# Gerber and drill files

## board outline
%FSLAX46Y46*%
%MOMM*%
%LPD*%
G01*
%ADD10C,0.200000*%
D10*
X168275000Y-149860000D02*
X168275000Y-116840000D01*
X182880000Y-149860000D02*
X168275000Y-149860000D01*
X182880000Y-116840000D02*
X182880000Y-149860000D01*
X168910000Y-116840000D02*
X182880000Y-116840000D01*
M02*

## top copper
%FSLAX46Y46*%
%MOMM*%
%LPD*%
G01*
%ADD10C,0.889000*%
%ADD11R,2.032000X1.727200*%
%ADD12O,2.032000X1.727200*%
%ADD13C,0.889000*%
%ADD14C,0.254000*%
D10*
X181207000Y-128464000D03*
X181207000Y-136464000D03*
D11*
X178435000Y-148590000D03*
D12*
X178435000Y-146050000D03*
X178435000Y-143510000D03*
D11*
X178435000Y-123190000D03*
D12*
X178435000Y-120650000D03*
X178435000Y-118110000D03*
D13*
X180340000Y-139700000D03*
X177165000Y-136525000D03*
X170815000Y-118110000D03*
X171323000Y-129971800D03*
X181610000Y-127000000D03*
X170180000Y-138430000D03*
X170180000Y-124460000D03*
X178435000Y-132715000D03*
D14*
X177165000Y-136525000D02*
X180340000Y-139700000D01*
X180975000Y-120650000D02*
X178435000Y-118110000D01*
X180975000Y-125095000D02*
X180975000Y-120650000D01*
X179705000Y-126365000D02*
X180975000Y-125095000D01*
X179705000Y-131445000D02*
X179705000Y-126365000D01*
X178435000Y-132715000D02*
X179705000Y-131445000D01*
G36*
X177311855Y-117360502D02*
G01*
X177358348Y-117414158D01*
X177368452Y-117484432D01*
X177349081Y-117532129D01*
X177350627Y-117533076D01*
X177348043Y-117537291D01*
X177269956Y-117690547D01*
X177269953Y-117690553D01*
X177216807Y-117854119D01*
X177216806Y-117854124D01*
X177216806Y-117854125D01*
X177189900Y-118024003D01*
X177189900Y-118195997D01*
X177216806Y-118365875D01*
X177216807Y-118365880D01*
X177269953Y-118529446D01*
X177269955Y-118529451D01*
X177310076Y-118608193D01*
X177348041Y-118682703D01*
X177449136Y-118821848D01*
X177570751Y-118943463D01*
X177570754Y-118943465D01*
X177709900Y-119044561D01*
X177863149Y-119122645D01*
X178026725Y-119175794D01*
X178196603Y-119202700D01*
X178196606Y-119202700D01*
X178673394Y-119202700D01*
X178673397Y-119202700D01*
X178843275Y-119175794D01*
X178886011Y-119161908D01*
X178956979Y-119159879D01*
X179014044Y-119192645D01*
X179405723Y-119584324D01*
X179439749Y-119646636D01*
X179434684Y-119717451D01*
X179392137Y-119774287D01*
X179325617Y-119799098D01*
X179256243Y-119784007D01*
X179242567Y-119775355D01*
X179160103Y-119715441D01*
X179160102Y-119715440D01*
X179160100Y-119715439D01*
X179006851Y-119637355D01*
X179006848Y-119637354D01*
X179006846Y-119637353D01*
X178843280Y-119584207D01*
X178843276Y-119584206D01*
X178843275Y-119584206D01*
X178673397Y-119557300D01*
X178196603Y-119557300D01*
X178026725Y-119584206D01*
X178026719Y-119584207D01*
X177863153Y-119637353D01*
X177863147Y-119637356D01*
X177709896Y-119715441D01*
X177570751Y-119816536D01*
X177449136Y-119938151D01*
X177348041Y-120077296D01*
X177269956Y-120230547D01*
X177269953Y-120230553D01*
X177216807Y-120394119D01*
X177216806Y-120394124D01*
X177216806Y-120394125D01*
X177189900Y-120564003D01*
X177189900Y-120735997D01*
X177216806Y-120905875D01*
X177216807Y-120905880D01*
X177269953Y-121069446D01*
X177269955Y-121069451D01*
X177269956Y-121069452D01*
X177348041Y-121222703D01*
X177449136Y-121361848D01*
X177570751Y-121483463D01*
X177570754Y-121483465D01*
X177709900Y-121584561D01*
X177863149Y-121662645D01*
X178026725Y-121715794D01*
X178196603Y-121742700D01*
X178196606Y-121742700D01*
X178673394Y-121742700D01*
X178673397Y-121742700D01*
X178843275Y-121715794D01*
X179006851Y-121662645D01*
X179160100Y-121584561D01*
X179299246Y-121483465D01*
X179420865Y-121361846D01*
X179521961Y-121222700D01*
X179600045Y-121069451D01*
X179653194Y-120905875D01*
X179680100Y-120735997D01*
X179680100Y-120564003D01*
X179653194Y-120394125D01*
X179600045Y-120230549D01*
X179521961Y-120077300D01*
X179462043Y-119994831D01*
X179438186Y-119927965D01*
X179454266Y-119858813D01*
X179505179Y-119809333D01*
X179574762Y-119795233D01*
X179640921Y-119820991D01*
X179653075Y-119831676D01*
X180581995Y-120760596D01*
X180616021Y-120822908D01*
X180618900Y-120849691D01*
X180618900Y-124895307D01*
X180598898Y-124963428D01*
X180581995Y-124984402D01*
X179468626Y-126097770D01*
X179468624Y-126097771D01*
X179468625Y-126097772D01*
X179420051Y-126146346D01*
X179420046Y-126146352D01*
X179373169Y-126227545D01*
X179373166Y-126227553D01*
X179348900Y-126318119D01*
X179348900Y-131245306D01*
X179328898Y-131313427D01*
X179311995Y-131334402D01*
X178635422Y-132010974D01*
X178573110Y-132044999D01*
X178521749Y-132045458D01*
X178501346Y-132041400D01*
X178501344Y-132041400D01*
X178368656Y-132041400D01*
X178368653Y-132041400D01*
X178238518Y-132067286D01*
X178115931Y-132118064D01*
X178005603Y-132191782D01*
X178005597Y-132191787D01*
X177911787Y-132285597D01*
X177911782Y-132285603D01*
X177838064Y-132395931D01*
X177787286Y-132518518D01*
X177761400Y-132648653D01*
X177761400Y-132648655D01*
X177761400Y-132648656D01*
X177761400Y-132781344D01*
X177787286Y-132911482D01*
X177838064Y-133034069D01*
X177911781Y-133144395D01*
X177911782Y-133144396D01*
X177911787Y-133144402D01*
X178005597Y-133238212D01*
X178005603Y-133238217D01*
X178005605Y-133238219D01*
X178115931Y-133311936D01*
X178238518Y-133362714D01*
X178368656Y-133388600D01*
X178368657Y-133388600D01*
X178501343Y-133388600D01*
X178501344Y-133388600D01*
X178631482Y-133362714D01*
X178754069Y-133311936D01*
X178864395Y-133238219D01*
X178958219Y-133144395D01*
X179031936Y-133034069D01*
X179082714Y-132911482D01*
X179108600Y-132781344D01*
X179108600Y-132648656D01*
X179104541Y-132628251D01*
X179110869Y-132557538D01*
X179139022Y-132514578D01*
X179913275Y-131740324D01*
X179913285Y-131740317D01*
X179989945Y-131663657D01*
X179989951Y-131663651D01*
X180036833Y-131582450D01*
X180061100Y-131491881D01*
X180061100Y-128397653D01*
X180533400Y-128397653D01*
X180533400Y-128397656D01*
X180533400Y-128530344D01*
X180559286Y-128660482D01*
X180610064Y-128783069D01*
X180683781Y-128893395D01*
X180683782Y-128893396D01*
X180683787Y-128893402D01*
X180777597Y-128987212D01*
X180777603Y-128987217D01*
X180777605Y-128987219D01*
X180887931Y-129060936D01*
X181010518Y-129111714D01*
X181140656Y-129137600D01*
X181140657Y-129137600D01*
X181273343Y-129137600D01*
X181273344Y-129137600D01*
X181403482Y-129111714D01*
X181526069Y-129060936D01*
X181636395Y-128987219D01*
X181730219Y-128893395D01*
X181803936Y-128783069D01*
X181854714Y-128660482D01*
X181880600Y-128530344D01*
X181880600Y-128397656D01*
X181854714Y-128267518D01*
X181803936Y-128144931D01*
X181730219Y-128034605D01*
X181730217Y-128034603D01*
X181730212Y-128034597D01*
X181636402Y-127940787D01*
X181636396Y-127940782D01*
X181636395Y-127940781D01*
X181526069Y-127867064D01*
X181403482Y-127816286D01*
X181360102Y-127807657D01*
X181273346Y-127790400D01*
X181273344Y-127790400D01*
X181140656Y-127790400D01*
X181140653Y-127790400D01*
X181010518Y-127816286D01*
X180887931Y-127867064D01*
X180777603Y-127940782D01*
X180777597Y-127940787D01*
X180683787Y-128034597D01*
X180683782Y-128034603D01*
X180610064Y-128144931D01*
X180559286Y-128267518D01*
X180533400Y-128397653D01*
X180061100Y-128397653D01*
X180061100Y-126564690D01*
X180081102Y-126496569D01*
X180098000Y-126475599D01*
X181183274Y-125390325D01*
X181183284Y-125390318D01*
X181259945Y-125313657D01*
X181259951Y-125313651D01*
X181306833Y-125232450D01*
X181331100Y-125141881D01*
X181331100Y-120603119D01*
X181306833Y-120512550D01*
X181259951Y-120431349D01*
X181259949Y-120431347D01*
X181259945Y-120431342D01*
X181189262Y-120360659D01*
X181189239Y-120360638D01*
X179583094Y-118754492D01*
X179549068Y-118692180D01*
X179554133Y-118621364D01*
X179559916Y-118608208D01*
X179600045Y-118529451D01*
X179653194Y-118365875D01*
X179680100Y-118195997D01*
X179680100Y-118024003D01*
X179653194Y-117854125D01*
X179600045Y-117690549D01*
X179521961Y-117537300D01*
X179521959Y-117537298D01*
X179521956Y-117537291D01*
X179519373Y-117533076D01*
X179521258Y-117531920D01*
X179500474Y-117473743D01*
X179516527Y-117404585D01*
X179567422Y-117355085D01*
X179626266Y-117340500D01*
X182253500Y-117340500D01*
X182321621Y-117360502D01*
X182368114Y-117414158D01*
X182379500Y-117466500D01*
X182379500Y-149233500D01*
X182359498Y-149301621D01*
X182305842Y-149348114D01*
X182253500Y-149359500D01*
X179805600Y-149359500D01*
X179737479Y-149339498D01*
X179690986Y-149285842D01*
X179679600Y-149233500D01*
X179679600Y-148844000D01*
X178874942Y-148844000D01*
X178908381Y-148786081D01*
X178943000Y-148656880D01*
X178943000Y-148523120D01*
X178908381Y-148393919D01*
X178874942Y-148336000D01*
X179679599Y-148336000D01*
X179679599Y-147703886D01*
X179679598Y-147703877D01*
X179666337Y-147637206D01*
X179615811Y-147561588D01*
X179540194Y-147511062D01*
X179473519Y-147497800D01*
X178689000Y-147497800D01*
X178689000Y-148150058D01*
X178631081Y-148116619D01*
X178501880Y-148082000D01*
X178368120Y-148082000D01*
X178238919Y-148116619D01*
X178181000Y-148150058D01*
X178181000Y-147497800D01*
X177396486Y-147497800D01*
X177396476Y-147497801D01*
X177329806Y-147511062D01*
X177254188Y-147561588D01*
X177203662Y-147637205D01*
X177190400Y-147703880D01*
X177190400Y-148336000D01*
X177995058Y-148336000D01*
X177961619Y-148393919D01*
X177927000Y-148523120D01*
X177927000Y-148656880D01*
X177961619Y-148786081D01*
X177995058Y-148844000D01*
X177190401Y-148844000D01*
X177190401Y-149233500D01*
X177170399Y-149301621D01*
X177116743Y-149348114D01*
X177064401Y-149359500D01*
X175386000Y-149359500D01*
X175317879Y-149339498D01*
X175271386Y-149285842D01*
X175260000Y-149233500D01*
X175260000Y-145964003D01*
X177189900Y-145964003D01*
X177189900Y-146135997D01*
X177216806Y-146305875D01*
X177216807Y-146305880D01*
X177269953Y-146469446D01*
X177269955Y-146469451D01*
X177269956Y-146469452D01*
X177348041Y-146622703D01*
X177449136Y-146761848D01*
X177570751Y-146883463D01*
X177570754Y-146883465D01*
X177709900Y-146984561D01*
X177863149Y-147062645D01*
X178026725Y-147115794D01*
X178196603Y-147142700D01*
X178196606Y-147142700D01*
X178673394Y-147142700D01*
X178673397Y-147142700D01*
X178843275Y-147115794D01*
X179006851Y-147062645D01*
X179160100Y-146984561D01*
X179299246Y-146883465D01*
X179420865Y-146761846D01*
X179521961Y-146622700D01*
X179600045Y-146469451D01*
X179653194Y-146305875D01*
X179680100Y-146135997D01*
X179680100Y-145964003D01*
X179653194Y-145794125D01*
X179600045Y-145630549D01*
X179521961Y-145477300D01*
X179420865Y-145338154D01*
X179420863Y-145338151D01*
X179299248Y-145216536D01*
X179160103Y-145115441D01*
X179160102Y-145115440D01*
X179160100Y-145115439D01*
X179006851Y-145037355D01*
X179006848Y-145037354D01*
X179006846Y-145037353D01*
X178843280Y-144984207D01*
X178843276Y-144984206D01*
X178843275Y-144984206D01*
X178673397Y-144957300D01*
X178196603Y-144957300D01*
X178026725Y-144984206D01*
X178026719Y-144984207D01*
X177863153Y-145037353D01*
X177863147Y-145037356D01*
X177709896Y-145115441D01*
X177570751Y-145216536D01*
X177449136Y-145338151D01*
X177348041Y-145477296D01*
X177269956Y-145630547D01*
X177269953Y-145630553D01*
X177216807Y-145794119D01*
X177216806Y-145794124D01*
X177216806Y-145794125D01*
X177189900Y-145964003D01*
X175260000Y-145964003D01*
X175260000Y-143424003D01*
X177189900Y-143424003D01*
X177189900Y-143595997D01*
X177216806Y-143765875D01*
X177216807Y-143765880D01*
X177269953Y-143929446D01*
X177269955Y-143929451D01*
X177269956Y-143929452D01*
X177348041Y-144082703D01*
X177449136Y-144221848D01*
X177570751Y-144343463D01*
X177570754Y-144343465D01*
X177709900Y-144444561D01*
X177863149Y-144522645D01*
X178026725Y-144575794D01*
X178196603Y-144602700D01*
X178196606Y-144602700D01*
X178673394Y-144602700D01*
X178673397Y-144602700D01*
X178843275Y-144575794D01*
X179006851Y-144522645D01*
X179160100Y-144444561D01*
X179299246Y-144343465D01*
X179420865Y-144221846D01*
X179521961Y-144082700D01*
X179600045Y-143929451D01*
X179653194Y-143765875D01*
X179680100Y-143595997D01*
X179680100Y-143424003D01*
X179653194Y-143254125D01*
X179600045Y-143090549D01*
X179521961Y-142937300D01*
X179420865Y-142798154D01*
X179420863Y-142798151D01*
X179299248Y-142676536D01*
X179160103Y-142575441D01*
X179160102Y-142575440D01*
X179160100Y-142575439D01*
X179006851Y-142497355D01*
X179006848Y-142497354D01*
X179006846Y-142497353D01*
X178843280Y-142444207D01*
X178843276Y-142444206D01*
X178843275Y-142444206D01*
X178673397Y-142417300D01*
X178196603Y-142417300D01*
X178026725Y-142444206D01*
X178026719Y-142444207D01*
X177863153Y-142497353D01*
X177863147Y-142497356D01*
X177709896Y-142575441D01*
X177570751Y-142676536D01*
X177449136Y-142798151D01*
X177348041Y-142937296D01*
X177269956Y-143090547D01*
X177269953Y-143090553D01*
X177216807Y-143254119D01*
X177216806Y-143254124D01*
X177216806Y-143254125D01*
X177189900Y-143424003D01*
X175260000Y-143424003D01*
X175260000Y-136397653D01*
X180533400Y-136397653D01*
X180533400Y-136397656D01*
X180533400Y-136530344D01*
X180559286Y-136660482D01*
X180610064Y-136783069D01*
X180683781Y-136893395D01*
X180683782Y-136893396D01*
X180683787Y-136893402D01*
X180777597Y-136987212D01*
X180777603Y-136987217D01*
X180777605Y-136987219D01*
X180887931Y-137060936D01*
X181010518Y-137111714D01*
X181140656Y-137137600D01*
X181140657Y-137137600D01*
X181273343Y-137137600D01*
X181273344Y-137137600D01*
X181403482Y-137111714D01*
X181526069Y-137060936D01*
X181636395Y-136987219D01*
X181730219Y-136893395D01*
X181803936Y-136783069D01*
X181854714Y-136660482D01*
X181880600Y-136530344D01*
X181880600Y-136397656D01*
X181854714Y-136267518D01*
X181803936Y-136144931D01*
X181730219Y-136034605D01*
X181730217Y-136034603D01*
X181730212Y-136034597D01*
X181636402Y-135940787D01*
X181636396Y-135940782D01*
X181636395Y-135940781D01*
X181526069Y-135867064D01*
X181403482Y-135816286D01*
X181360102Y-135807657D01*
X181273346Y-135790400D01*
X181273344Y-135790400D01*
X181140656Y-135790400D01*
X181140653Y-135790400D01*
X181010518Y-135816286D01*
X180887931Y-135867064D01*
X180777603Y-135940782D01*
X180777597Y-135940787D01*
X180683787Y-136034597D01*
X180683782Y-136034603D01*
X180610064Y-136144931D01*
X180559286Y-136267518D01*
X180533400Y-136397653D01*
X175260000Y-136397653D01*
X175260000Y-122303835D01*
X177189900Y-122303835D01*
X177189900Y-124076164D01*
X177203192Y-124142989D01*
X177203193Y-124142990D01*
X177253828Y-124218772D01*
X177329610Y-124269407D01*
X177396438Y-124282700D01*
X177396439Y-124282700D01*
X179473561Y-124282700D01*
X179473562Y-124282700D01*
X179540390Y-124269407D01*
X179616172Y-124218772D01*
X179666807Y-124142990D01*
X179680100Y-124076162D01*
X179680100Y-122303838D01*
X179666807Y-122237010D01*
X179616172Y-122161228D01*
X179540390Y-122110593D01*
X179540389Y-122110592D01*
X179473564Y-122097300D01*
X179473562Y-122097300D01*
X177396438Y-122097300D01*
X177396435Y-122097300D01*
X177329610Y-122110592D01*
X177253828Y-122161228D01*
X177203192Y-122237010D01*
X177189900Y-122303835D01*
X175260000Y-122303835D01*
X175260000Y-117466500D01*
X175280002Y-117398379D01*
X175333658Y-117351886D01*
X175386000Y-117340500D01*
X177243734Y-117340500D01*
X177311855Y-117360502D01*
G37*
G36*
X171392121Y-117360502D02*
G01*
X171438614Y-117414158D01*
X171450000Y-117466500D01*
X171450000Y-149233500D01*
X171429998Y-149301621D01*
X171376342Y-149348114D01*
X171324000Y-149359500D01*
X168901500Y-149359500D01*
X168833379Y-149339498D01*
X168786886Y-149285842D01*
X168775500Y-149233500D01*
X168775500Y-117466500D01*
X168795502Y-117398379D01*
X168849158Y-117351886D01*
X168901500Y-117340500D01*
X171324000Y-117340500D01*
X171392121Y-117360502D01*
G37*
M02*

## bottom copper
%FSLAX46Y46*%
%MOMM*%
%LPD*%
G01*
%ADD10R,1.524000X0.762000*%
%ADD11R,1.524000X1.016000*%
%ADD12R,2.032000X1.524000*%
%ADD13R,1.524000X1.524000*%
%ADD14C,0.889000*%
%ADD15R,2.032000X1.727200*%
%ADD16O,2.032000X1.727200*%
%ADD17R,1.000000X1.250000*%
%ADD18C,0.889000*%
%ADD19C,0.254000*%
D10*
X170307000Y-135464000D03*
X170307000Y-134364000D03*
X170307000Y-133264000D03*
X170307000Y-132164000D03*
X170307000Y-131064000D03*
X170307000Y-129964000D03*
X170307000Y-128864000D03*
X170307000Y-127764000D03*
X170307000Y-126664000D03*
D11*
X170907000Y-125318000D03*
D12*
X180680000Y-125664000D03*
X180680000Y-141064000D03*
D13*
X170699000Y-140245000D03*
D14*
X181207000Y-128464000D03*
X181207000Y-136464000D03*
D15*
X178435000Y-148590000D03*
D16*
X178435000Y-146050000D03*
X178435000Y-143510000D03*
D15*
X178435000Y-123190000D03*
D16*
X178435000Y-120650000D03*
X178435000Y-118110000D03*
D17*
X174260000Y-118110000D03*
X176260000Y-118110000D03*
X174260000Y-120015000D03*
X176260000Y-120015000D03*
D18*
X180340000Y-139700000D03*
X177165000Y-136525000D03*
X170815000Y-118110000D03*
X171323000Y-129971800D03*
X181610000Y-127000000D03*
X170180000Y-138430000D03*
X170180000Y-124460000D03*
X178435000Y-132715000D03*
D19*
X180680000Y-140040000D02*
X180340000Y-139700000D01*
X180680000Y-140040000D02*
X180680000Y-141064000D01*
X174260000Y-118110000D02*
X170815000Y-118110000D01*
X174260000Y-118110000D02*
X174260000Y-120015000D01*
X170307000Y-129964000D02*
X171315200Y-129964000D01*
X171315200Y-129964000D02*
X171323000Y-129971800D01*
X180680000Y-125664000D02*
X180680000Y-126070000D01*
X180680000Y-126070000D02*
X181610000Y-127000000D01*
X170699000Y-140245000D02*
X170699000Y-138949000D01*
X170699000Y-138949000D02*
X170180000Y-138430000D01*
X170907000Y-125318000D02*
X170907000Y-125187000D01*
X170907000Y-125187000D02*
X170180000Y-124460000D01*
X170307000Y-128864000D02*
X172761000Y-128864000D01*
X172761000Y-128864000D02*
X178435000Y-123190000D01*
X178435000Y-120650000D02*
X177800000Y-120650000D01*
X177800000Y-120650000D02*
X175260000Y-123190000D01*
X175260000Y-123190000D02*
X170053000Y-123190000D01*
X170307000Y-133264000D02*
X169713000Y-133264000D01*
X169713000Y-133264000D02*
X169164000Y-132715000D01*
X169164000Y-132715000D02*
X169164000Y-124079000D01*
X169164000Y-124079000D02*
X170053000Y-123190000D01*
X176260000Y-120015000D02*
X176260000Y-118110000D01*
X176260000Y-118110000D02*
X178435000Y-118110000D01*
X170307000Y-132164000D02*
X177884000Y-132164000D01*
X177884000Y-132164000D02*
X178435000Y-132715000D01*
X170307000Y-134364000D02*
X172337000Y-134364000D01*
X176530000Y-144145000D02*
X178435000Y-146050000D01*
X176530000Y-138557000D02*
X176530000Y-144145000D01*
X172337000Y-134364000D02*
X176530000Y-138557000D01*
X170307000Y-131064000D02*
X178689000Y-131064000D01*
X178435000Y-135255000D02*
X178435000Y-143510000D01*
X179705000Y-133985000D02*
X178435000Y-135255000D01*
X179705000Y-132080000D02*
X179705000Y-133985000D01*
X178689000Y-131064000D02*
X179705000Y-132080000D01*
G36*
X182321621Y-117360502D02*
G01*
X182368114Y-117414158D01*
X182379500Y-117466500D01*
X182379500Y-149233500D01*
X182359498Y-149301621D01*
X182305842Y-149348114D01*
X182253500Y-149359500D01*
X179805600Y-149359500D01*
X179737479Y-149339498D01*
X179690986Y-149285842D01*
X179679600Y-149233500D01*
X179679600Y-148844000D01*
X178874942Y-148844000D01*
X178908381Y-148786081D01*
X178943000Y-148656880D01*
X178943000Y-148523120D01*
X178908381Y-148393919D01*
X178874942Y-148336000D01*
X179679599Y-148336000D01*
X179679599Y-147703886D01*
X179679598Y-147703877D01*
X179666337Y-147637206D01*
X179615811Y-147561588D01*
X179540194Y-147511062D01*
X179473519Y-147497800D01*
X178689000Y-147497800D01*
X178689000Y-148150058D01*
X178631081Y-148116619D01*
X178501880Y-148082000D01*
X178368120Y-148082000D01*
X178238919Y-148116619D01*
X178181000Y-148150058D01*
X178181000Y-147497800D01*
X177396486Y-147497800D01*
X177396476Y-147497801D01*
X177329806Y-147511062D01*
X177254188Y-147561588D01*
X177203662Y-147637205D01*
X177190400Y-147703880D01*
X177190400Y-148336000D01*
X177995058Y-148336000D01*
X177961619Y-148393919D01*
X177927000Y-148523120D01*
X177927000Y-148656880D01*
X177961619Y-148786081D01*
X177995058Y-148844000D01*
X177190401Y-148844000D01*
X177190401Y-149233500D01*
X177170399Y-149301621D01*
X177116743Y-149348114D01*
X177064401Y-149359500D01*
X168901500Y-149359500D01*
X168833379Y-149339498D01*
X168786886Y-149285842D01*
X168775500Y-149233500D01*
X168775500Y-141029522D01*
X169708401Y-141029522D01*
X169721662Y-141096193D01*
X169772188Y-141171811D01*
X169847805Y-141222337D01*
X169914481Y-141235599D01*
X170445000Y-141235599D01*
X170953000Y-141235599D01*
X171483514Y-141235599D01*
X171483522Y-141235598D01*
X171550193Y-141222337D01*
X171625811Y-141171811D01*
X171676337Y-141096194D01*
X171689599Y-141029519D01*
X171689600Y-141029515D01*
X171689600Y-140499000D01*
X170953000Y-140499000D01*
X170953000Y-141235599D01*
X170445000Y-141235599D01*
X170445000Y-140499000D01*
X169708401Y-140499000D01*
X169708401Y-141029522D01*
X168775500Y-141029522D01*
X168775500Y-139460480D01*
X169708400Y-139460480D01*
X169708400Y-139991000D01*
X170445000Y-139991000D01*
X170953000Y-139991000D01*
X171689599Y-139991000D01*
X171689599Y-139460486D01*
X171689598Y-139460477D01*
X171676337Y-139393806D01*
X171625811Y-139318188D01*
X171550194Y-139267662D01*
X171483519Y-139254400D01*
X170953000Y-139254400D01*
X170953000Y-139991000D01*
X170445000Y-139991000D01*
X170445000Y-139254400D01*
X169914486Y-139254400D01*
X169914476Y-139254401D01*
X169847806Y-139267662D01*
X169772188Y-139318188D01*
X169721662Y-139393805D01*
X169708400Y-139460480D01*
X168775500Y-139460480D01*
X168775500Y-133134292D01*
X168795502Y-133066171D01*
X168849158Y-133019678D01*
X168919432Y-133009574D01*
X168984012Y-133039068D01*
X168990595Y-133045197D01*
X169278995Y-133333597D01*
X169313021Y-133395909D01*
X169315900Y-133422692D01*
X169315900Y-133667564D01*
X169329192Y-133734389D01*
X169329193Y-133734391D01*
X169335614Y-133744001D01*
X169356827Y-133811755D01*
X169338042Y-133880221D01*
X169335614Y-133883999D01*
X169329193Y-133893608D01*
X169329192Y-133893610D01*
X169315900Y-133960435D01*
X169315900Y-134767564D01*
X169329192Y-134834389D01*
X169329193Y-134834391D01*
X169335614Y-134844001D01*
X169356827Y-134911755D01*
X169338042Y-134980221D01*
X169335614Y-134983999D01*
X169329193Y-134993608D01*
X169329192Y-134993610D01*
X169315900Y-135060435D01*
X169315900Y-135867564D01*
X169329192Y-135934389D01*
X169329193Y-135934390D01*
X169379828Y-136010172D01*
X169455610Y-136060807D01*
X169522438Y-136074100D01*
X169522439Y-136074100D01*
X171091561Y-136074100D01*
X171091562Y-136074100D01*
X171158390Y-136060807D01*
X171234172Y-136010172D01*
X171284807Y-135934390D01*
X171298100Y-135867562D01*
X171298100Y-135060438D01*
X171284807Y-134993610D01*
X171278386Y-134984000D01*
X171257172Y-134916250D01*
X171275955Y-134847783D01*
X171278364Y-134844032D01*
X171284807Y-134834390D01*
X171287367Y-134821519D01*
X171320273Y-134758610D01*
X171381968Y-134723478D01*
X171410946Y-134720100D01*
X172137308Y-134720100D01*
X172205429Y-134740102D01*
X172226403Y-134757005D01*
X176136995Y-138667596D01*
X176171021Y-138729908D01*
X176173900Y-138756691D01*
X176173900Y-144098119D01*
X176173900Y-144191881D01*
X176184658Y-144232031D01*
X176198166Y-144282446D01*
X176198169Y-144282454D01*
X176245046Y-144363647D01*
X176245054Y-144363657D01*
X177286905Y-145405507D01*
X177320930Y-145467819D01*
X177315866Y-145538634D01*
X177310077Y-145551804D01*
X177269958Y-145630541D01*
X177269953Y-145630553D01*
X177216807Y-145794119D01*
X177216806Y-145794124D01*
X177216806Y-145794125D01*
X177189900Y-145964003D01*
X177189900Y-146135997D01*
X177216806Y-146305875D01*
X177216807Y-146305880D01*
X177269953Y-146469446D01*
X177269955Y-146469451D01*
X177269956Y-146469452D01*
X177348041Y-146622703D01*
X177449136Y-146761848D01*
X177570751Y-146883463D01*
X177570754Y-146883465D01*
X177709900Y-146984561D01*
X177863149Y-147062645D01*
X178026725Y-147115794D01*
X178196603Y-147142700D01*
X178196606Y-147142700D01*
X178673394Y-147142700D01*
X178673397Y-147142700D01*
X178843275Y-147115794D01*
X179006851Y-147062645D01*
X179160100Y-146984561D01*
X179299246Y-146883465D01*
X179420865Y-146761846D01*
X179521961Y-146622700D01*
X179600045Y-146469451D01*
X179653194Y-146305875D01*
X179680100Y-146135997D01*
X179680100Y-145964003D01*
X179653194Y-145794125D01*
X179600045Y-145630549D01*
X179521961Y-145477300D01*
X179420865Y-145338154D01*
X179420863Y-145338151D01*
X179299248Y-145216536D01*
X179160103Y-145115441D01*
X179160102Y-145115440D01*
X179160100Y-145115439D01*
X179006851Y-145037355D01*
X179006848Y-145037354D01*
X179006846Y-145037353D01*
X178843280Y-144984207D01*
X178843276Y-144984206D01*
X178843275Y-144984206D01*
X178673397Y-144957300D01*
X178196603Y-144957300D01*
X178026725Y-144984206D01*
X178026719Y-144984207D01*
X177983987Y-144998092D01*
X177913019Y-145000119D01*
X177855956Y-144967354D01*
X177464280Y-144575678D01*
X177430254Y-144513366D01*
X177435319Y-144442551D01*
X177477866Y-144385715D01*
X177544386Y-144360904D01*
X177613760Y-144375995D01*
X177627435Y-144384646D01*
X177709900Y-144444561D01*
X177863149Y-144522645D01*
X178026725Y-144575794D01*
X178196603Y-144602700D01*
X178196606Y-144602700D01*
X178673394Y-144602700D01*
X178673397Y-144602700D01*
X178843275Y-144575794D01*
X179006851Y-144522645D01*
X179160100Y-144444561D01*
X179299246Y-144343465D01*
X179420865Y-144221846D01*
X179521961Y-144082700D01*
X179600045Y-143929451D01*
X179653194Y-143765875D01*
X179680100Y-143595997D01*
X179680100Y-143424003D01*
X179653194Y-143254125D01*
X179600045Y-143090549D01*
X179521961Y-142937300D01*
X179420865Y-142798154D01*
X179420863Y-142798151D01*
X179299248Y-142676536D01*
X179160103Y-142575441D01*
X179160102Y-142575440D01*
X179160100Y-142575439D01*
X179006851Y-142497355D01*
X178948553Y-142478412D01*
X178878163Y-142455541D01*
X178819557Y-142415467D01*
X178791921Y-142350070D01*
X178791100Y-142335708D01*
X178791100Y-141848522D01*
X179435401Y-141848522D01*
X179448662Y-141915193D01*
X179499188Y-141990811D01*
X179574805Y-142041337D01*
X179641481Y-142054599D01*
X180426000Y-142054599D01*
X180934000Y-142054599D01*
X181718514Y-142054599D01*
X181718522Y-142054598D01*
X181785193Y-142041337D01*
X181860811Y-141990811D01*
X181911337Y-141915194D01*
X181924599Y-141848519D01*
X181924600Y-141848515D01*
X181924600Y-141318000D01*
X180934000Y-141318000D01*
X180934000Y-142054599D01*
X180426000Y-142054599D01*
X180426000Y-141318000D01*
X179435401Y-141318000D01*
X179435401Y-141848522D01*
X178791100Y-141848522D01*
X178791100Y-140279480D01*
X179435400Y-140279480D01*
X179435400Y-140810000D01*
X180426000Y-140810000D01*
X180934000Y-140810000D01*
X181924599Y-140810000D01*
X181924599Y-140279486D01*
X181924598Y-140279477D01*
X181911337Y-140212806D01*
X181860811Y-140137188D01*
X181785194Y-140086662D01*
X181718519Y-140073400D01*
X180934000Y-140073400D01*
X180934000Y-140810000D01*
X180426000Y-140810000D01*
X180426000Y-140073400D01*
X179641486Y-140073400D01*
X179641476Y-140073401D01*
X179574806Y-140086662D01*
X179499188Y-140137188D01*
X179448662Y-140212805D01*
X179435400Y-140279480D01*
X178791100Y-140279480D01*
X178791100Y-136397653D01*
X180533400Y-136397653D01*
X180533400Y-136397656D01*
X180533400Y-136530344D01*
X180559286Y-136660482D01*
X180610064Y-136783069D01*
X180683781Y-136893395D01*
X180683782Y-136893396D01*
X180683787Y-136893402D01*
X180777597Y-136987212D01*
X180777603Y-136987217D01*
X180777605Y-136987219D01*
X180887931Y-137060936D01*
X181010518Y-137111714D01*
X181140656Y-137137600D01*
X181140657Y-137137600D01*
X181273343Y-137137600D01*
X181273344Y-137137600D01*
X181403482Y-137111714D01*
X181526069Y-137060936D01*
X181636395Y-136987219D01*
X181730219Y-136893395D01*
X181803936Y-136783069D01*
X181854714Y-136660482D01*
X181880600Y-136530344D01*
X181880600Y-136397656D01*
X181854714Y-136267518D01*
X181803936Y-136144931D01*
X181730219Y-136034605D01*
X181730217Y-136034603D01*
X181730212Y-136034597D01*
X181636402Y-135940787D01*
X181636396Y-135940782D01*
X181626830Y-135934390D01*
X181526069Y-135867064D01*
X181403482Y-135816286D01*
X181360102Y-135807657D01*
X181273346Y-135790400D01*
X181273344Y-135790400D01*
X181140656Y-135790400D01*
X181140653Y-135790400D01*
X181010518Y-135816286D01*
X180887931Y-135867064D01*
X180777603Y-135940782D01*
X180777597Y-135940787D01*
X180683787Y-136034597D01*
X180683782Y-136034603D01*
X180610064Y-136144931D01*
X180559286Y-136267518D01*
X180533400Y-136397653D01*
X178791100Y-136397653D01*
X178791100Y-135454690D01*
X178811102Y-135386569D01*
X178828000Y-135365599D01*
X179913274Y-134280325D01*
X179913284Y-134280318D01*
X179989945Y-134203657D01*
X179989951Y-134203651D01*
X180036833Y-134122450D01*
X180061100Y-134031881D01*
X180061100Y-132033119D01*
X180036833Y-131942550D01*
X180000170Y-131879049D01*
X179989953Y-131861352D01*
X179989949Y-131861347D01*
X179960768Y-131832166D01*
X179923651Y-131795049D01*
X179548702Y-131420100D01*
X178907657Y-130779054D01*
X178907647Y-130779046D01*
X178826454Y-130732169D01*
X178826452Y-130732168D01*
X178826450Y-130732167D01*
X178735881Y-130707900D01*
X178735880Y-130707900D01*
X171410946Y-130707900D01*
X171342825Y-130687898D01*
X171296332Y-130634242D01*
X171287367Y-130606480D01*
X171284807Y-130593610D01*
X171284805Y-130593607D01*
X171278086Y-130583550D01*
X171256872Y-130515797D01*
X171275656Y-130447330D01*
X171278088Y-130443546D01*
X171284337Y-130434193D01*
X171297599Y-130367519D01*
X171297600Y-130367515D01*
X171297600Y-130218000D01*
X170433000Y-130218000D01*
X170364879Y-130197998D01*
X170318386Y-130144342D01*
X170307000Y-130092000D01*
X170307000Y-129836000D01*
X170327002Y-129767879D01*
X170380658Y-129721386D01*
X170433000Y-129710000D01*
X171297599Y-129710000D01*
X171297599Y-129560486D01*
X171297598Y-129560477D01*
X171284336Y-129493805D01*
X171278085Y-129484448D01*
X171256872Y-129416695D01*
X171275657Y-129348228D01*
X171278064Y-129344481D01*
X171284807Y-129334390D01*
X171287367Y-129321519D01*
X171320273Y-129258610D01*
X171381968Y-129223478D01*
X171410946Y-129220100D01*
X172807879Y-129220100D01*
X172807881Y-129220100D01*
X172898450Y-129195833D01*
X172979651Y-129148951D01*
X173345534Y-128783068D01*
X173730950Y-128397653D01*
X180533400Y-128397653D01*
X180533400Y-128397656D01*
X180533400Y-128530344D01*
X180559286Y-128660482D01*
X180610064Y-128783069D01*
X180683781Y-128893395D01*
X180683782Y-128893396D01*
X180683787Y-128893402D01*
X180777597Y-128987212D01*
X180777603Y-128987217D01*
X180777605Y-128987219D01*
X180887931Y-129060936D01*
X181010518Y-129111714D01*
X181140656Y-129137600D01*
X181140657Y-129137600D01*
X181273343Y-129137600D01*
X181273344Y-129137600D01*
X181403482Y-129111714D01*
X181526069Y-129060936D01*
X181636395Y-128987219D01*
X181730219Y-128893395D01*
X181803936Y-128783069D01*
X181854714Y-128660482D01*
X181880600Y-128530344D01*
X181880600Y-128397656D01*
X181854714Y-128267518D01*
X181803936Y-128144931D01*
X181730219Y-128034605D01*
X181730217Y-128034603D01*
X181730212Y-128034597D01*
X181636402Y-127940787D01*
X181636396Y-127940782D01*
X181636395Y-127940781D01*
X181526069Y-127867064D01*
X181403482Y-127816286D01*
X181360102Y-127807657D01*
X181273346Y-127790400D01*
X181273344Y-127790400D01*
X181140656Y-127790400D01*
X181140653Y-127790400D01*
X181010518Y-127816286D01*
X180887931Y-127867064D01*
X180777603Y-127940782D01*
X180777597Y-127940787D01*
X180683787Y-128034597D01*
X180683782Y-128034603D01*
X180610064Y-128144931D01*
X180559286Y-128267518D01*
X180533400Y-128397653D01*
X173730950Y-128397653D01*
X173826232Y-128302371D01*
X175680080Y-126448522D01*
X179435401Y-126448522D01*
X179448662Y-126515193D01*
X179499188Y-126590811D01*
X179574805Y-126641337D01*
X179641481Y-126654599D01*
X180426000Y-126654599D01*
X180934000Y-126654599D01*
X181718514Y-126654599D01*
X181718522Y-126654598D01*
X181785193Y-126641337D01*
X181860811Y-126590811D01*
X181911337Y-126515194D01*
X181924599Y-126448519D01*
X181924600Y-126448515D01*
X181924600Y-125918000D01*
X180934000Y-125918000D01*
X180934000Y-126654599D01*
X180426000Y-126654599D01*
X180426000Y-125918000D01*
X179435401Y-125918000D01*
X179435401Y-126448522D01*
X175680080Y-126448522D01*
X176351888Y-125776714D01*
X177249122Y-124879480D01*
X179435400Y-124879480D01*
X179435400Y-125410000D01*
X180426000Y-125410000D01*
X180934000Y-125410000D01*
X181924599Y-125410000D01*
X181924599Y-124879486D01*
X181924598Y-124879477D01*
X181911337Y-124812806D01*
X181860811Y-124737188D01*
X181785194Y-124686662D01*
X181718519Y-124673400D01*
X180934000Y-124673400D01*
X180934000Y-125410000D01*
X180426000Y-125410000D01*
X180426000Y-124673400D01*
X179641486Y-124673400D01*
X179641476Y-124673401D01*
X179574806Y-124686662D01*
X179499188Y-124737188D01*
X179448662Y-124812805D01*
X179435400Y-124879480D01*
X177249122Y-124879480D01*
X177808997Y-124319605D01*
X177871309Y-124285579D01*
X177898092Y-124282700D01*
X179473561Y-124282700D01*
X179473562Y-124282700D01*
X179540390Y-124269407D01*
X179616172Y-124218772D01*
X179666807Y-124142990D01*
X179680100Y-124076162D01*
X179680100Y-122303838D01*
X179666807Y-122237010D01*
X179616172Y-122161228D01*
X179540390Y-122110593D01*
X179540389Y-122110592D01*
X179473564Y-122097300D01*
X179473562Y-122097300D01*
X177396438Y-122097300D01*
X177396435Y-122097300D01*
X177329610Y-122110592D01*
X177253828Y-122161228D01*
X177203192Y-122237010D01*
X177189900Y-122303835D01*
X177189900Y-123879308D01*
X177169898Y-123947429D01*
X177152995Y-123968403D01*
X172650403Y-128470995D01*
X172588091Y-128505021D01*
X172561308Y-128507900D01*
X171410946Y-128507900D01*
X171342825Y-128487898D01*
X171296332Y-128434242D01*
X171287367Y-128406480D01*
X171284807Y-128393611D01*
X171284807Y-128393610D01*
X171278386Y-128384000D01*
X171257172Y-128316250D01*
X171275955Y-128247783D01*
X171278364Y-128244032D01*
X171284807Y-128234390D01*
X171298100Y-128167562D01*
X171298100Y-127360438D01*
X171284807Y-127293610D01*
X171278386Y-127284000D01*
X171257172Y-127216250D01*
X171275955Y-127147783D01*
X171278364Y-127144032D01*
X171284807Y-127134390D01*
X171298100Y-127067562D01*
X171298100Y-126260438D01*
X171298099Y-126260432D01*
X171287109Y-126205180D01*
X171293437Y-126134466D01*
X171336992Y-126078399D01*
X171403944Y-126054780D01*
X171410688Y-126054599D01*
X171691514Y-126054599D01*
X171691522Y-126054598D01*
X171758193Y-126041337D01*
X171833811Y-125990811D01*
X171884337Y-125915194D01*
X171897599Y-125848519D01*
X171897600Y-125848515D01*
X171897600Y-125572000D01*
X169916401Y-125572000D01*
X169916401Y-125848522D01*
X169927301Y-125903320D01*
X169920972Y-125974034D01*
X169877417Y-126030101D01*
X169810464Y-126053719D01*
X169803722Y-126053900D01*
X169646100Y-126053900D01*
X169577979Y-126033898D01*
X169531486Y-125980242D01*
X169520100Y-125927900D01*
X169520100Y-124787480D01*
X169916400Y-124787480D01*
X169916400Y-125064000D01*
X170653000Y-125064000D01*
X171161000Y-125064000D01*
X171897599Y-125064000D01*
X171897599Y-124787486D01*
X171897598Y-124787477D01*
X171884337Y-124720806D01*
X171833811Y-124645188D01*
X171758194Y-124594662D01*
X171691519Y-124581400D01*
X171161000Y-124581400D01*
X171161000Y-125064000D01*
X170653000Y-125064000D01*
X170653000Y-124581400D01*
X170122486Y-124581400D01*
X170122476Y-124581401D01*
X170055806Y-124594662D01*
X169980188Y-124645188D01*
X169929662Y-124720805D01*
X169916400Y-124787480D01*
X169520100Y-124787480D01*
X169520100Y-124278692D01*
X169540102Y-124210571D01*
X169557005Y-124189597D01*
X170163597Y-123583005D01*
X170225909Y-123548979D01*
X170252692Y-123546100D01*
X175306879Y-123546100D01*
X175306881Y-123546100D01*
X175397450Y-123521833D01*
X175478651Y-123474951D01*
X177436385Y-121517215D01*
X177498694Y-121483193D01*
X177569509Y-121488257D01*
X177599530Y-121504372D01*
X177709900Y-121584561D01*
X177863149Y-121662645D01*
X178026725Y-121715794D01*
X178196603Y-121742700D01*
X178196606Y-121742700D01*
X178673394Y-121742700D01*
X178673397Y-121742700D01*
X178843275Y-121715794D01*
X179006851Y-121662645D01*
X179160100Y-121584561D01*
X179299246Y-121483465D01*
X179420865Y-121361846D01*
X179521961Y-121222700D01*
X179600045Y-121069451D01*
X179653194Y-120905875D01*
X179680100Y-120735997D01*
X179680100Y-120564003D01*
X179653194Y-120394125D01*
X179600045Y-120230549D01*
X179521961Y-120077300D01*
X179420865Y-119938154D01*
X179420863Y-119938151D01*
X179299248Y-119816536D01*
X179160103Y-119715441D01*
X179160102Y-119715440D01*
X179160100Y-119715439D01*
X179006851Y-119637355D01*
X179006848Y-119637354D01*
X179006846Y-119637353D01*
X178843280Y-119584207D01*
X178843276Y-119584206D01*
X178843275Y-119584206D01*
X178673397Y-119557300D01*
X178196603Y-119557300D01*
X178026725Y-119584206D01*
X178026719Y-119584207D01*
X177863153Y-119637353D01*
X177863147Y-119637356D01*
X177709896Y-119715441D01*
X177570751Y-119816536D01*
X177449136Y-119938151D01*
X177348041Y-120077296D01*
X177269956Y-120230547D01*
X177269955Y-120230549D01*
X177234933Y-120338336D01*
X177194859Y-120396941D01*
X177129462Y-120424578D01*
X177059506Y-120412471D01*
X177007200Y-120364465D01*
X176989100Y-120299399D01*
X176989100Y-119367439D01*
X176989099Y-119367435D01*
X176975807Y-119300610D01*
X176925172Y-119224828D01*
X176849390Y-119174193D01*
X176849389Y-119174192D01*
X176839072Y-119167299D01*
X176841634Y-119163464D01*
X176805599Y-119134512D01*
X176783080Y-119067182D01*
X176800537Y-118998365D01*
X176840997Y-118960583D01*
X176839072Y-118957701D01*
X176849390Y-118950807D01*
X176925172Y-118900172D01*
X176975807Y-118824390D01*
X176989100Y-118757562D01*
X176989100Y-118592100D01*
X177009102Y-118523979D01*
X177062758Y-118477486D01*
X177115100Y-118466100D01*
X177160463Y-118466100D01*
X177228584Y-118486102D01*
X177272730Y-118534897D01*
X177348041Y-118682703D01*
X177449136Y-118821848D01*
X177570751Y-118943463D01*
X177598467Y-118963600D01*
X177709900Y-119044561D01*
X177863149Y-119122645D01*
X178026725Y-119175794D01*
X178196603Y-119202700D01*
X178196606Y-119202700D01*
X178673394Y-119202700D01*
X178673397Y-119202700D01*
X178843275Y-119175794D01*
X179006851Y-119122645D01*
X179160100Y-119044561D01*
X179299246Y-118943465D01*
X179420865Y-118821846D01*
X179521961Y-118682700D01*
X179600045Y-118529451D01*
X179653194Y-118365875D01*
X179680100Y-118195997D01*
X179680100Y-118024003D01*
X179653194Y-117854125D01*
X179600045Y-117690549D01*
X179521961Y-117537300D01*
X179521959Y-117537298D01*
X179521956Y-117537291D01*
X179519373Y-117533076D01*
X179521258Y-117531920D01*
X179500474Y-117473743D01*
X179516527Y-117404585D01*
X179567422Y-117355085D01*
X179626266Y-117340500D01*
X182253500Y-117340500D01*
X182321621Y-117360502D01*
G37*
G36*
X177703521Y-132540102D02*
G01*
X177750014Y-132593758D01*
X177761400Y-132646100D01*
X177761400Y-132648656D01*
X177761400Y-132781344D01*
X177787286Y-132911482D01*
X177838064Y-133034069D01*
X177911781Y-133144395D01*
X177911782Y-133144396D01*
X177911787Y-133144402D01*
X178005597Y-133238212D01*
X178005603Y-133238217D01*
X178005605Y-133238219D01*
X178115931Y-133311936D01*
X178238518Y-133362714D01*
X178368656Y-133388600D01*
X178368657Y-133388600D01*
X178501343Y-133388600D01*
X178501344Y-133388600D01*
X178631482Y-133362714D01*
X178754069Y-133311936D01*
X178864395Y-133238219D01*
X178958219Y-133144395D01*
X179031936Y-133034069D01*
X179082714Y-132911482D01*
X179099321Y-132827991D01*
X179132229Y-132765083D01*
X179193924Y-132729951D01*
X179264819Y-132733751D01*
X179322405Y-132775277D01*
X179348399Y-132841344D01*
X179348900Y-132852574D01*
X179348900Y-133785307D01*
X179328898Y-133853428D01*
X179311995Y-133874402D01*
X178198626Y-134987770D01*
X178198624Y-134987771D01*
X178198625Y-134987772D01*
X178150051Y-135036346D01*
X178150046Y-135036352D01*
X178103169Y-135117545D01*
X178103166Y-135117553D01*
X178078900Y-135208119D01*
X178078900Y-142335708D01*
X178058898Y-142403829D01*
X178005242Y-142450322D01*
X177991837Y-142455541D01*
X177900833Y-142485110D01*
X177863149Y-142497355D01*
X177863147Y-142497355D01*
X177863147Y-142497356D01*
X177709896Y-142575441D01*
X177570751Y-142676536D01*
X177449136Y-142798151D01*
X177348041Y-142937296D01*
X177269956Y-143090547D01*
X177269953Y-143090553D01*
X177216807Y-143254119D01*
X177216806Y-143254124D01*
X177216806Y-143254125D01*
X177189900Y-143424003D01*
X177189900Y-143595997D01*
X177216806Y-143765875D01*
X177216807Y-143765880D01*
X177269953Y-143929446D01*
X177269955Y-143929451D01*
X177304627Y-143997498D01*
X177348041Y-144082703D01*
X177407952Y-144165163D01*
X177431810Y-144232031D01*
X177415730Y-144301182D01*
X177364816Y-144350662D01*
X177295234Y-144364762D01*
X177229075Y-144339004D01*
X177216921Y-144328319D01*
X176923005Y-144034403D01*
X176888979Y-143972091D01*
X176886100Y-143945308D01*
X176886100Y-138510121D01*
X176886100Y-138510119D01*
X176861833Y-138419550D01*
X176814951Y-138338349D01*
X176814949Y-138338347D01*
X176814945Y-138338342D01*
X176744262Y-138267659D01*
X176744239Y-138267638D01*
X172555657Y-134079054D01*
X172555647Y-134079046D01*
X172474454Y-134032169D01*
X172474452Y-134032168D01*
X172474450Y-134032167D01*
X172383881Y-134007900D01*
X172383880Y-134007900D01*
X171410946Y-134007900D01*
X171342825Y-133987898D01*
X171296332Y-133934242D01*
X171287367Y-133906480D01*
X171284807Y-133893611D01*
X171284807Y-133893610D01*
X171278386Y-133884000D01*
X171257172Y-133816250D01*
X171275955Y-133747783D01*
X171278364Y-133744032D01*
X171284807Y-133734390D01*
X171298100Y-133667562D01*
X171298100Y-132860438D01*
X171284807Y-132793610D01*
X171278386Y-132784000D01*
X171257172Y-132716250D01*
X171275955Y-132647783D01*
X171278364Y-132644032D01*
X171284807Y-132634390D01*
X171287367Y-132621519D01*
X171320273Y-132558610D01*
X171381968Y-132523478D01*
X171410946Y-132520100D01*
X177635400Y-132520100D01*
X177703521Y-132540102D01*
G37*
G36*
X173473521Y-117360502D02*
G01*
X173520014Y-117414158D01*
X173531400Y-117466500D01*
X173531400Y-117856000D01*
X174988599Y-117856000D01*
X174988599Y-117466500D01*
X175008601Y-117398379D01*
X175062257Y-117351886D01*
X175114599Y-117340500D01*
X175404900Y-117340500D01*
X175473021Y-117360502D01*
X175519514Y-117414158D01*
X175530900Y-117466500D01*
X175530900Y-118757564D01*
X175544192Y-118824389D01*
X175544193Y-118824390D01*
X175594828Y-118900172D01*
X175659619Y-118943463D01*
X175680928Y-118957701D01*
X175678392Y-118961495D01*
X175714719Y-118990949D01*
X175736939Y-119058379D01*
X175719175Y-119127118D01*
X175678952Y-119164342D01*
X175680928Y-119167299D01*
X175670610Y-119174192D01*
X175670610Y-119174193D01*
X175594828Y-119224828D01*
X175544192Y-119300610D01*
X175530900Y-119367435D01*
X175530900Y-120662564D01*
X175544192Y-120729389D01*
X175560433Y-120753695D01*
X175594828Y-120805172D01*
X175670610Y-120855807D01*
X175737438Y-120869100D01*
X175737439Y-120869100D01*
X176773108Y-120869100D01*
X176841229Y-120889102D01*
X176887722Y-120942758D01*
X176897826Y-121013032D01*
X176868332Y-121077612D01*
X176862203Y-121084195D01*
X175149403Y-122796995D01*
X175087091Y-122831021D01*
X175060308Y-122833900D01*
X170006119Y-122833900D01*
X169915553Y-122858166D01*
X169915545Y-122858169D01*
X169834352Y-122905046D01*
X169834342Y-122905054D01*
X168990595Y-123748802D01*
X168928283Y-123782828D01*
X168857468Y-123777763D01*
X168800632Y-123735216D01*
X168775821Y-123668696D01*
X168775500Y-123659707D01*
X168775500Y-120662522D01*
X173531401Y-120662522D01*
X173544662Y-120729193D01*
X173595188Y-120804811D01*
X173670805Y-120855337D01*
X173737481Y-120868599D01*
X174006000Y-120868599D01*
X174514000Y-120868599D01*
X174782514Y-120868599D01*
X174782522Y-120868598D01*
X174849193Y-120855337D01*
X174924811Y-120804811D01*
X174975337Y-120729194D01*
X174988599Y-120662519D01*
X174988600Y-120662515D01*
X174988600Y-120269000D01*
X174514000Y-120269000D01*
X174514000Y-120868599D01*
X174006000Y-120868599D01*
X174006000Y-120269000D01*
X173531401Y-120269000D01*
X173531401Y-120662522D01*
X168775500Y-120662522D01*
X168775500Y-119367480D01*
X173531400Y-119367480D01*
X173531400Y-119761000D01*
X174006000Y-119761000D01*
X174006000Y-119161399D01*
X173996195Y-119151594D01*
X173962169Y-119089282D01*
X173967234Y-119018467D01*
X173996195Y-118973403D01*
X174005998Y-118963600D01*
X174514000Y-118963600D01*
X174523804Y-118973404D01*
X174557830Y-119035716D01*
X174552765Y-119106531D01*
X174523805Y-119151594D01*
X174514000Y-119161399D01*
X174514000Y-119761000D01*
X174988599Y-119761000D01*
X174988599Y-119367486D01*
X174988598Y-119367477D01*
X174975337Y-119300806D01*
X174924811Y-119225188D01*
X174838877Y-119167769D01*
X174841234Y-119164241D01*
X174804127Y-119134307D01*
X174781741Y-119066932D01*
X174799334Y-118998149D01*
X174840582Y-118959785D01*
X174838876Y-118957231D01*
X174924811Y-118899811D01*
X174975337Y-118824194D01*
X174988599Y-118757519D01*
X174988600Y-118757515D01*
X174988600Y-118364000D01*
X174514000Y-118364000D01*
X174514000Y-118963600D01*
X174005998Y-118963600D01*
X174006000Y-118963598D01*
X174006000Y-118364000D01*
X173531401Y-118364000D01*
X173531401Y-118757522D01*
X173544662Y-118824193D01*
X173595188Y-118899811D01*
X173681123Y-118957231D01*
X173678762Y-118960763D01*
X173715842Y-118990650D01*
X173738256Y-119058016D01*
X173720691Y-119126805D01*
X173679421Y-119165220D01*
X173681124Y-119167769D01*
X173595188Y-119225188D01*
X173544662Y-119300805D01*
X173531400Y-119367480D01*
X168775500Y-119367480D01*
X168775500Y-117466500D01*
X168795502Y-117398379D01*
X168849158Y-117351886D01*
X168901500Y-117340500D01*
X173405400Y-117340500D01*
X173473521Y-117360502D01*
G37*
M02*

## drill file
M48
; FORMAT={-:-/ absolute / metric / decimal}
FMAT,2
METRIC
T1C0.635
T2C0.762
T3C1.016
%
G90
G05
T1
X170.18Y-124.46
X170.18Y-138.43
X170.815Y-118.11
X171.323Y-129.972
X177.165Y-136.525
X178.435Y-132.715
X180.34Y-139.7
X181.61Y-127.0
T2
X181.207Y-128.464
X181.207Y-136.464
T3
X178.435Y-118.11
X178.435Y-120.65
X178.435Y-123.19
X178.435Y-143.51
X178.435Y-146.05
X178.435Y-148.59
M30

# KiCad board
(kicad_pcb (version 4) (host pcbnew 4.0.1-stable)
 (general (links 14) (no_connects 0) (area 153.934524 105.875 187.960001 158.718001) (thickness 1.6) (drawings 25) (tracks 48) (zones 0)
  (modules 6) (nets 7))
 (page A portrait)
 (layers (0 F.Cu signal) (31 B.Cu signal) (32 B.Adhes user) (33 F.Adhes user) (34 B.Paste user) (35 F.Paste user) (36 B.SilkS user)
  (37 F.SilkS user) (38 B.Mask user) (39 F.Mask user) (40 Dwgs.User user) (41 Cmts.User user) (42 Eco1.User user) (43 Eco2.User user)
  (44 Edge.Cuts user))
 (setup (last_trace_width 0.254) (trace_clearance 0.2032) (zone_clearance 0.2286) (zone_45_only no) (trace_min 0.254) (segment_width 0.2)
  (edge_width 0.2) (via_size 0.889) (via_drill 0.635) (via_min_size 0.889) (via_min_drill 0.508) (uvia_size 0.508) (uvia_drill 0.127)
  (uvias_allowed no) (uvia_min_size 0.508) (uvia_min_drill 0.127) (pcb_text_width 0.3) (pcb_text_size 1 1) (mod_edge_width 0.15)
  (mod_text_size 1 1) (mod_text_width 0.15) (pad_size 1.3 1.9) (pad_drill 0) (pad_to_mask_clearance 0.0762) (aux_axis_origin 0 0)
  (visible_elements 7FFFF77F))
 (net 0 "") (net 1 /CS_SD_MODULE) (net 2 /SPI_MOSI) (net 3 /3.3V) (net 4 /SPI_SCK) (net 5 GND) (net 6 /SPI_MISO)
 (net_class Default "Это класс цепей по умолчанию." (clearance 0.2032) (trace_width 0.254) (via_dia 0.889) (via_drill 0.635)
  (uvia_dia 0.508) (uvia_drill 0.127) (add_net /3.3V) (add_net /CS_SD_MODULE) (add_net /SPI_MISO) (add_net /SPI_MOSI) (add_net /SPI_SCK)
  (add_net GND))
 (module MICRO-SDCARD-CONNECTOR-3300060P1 (layer B.Cu) (at 177.8 133.35)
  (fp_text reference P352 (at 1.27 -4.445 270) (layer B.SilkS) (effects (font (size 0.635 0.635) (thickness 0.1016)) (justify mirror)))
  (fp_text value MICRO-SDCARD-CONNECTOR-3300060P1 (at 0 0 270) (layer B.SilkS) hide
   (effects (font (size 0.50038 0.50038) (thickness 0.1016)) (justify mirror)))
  (pad 1 smd rect (at -7.493 2.114) (size 1.524 0.762) (layers B.Cu B.Paste B.Mask))
  (pad 2 smd rect (at -7.493 1.014) (size 1.524 0.762) (layers B.Cu B.Paste B.Mask) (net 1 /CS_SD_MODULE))
  (pad 3 smd rect (at -7.493 -0.086) (size 1.524 0.762) (layers B.Cu B.Paste B.Mask) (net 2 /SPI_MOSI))
  (pad 4 smd rect (at -7.493 -1.186) (size 1.524 0.762) (layers B.Cu B.Paste B.Mask) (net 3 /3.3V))
  (pad 5 smd rect (at -7.493 -2.286) (size 1.524 0.762) (layers B.Cu B.Paste B.Mask) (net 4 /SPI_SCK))
  (pad 6 smd rect (at -7.493 -3.386) (size 1.524 0.762) (layers B.Cu B.Paste B.Mask) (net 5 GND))
  (pad 7 smd rect (at -7.493 -4.486) (size 1.524 0.762) (layers B.Cu B.Paste B.Mask) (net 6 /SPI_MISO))
  (pad 8 smd rect (at -7.493 -5.586) (size 1.524 0.762) (layers B.Cu B.Paste B.Mask))
  (pad 9 smd rect (at -7.493 -6.686) (size 1.524 0.762) (layers B.Cu B.Paste B.Mask))
  (pad G1 smd rect (at -6.893 -8.032) (size 1.524 1.016) (layers B.Cu B.Paste B.Mask) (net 5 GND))
  (pad G2 smd rect (at 2.88 -7.686) (size 2.032 1.524) (layers B.Cu B.Paste B.Mask) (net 5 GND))
  (pad G3 smd rect (at 2.88 7.714) (size 2.032 1.524) (layers B.Cu B.Paste B.Mask) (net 5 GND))
  (pad G4 smd rect (at -7.101 6.895) (size 1.524 1.524) (layers B.Cu B.Paste B.Mask) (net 5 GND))
  (pad "" thru_hole circle (at 3.407 -4.886) (size 0.889 0.889) (drill 0.762) (layers *.Cu *.Mask B.SilkS))
  (pad "" thru_hole circle (at 3.407 3.114) (size 0.889 0.889) (drill 0.762) (layers *.Cu *.Mask B.SilkS)))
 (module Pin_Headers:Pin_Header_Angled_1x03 (layer F.Cu) (at 178.435 148.59 180)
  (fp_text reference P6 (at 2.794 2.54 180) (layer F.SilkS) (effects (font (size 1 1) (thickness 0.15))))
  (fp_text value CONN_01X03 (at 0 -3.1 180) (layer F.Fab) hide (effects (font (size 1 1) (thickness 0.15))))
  (pad 1 thru_hole rect (at 0 0 180) (size 2.032 1.7272) (drill 1.016) (layers *.Cu *.Mask) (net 5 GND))
  (pad 2 thru_hole oval (at 0 2.54 180) (size 2.032 1.7272) (drill 1.016) (layers *.Cu *.Mask) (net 1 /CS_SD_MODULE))
  (pad 3 thru_hole oval (at 0 5.08 180) (size 2.032 1.7272) (drill 1.016) (layers *.Cu *.Mask) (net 4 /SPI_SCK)))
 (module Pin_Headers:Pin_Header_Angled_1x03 (layer F.Cu) (at 178.435 123.19 180)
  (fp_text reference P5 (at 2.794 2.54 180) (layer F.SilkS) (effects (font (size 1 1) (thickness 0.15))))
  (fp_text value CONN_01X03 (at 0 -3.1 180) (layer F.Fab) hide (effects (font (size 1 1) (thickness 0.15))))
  (pad 1 thru_hole rect (at 0 0 180) (size 2.032 1.7272) (drill 1.016) (layers *.Cu *.Mask) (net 6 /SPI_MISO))
  (pad 2 thru_hole oval (at 0 2.54 180) (size 2.032 1.7272) (drill 1.016) (layers *.Cu *.Mask) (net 2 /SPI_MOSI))
  (pad 3 thru_hole oval (at 0 5.08 180) (size 2.032 1.7272) (drill 1.016) (layers *.Cu *.Mask) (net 3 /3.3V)))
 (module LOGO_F (layer F.Cu) (at 175.895 137.16)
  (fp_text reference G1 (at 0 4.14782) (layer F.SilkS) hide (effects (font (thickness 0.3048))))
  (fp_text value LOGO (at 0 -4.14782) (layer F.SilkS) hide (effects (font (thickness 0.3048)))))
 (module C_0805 (layer B.Cu) (at 175.26 118.11)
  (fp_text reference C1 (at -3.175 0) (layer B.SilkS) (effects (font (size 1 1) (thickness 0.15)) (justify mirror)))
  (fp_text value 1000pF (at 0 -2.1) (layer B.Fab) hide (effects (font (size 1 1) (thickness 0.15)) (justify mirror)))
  (pad 1 smd rect (at -1 0) (size 1 1.25) (layers B.Cu B.Paste B.Mask) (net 5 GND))
  (pad 2 smd rect (at 1 0) (size 1 1.25) (layers B.Cu B.Paste B.Mask) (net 3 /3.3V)))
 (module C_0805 (layer B.Cu) (at 175.26 120.015)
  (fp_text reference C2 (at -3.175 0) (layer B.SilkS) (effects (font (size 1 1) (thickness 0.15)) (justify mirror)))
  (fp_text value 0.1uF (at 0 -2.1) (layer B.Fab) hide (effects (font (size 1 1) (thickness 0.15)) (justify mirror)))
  (pad 1 smd rect (at -1 0) (size 1 1.25) (layers B.Cu B.Paste B.Mask) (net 5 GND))
  (pad 2 smd rect (at 1 0) (size 1 1.25) (layers B.Cu B.Paste B.Mask) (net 3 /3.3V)))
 (gr_line (start 168.275 149.86) (end 168.275 116.84) (angle 90) (layer Edge.Cuts) (width 0.2))
 (gr_line (start 182.88 149.86) (end 168.275 149.86) (angle 90) (layer Edge.Cuts) (width 0.2))
 (gr_line (start 182.88 116.84) (end 182.88 149.86) (angle 90) (layer Edge.Cuts) (width 0.2))
 (gr_line (start 168.91 116.84) (end 182.88 116.84) (angle 90) (layer Edge.Cuts) (width 0.2))
 (segment (start 177.165 136.525) (end 180.34 139.7) (width 0.254) (layer F.Cu) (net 5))
 (segment (start 180.68 140.04) (end 180.34 139.7) (width 0.254) (layer B.Cu) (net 5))
 (via (at 180.34 139.7) (size 0.889) (drill 0.635) (layers F.Cu B.Cu) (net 5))
 (segment (start 180.68 140.04) (end 180.68 141.064) (width 0.254) (layer B.Cu) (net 5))
 (via (at 177.165 136.525) (size 0.889) (drill 0.635) (layers F.Cu B.Cu) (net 5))
 (segment (start 174.26 118.11) (end 170.815 118.11) (width 0.254) (layer B.Cu) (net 5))
 (via (at 170.815 118.11) (size 0.889) (drill 0.635) (layers F.Cu B.Cu) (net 5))
 (segment (start 174.26 118.11) (end 174.26 120.015) (width 0.254) (layer B.Cu) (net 5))
 (segment (start 170.307 129.964) (end 171.3152 129.964) (width 0.254) (layer B.Cu) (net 5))
 (via (at 171.323 129.9718) (size 0.889) (drill 0.635) (layers F.Cu B.Cu) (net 5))
 (segment (start 171.3152 129.964) (end 171.323 129.9718) (width 0.254) (layer B.Cu) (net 5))
 (segment (start 180.68 125.664) (end 180.68 126.07) (width 0.254) (layer B.Cu) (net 5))
 (segment (start 180.68 126.07) (end 181.61 127) (width 0.254) (layer B.Cu) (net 5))
 (via (at 181.61 127) (size 0.889) (drill 0.635) (layers F.Cu B.Cu) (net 5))
 (segment (start 170.699 140.245) (end 170.699 138.949) (width 0.254) (layer B.Cu) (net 5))
 (via (at 170.18 138.43) (size 0.889) (drill 0.635) (layers F.Cu B.Cu) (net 5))
 (segment (start 170.699 138.949) (end 170.18 138.43) (width 0.254) (layer B.Cu) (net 5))
 (segment (start 170.907 125.318) (end 170.907 125.187) (width 0.254) (layer B.Cu) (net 5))
 (segment (start 170.907 125.187) (end 170.18 124.46) (width 0.254) (layer B.Cu) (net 5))
 (via (at 170.18 124.46) (size 0.889) (drill 0.635) (layers F.Cu B.Cu) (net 5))
 (segment (start 170.307 128.864) (end 172.761 128.864) (width 0.254) (layer B.Cu) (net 6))
 (segment (start 172.761 128.864) (end 178.435 123.19) (width 0.254) (layer B.Cu) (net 6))
 (segment (start 178.435 120.65) (end 177.8 120.65) (width 0.254) (layer B.Cu) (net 2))
 (segment (start 177.8 120.65) (end 175.26 123.19) (width 0.254) (layer B.Cu) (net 2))
 (segment (start 175.26 123.19) (end 170.053 123.19) (width 0.254) (layer B.Cu) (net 2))
 (segment (start 170.307 133.264) (end 169.713 133.264) (width 0.254) (layer B.Cu) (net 2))
 (segment (start 169.713 133.264) (end 169.164 132.715) (width 0.254) (layer B.Cu) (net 2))
 (segment (start 169.164 132.715) (end 169.164 124.079) (width 0.254) (layer B.Cu) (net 2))
 (segment (start 169.164 124.079) (end 170.053 123.19) (width 0.254) (layer B.Cu) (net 2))
 (segment (start 176.26 120.015) (end 176.26 118.11) (width 0.254) (layer B.Cu) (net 3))
 (segment (start 176.26 118.11) (end 178.435 118.11) (width 0.254) (layer B.Cu) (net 3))
 (segment (start 170.307 132.164) (end 177.884 132.164) (width 0.254) (layer B.Cu) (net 3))
 (segment (start 180.975 120.65) (end 178.435 118.11) (width 0.254) (layer F.Cu) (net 3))
 (segment (start 180.975 125.095) (end 180.975 120.65) (width 0.254) (layer F.Cu) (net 3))
 (segment (start 179.705 126.365) (end 180.975 125.095) (width 0.254) (layer F.Cu) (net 3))
 (segment (start 179.705 131.445) (end 179.705 126.365) (width 0.254) (layer F.Cu) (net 3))
 (segment (start 178.435 132.715) (end 179.705 131.445) (width 0.254) (layer F.Cu) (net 3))
 (via (at 178.435 132.715) (size 0.889) (drill 0.635) (layers F.Cu B.Cu) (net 3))
 (segment (start 177.884 132.164) (end 178.435 132.715) (width 0.254) (layer B.Cu) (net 3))
 (segment (start 170.307 134.364) (end 172.337 134.364) (width 0.254) (layer B.Cu) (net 1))
 (segment (start 176.53 144.145) (end 178.435 146.05) (width 0.254) (layer B.Cu) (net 1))
 (segment (start 176.53 138.557) (end 176.53 144.145) (width 0.254) (layer B.Cu) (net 1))
 (segment (start 172.337 134.364) (end 176.53 138.557) (width 0.254) (layer B.Cu) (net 1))
 (segment (start 170.307 131.064) (end 178.689 131.064) (width 0.254) (layer B.Cu) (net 4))
 (segment (start 178.435 135.255) (end 178.435 143.51) (width 0.254) (layer B.Cu) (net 4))
 (segment (start 179.705 133.985) (end 178.435 135.255) (width 0.254) (layer B.Cu) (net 4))
 (segment (start 179.705 132.08) (end 179.705 133.985) (width 0.254) (layer B.Cu) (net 4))
 (segment (start 178.689 131.064) (end 179.705 132.08) (width 0.254) (layer B.Cu) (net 4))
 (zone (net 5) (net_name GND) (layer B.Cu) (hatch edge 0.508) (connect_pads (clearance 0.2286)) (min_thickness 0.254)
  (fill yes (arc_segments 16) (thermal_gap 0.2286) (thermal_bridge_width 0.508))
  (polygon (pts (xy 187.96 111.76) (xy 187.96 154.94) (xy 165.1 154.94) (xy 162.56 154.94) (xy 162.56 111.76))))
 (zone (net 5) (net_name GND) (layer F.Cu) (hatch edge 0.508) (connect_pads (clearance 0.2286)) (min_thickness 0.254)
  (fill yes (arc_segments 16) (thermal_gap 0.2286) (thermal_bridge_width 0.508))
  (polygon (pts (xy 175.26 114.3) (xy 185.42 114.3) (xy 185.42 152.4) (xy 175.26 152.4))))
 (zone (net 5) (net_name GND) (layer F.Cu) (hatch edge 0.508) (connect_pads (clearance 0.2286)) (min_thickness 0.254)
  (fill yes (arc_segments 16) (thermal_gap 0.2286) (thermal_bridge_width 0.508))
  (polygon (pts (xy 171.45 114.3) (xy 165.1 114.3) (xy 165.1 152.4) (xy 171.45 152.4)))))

